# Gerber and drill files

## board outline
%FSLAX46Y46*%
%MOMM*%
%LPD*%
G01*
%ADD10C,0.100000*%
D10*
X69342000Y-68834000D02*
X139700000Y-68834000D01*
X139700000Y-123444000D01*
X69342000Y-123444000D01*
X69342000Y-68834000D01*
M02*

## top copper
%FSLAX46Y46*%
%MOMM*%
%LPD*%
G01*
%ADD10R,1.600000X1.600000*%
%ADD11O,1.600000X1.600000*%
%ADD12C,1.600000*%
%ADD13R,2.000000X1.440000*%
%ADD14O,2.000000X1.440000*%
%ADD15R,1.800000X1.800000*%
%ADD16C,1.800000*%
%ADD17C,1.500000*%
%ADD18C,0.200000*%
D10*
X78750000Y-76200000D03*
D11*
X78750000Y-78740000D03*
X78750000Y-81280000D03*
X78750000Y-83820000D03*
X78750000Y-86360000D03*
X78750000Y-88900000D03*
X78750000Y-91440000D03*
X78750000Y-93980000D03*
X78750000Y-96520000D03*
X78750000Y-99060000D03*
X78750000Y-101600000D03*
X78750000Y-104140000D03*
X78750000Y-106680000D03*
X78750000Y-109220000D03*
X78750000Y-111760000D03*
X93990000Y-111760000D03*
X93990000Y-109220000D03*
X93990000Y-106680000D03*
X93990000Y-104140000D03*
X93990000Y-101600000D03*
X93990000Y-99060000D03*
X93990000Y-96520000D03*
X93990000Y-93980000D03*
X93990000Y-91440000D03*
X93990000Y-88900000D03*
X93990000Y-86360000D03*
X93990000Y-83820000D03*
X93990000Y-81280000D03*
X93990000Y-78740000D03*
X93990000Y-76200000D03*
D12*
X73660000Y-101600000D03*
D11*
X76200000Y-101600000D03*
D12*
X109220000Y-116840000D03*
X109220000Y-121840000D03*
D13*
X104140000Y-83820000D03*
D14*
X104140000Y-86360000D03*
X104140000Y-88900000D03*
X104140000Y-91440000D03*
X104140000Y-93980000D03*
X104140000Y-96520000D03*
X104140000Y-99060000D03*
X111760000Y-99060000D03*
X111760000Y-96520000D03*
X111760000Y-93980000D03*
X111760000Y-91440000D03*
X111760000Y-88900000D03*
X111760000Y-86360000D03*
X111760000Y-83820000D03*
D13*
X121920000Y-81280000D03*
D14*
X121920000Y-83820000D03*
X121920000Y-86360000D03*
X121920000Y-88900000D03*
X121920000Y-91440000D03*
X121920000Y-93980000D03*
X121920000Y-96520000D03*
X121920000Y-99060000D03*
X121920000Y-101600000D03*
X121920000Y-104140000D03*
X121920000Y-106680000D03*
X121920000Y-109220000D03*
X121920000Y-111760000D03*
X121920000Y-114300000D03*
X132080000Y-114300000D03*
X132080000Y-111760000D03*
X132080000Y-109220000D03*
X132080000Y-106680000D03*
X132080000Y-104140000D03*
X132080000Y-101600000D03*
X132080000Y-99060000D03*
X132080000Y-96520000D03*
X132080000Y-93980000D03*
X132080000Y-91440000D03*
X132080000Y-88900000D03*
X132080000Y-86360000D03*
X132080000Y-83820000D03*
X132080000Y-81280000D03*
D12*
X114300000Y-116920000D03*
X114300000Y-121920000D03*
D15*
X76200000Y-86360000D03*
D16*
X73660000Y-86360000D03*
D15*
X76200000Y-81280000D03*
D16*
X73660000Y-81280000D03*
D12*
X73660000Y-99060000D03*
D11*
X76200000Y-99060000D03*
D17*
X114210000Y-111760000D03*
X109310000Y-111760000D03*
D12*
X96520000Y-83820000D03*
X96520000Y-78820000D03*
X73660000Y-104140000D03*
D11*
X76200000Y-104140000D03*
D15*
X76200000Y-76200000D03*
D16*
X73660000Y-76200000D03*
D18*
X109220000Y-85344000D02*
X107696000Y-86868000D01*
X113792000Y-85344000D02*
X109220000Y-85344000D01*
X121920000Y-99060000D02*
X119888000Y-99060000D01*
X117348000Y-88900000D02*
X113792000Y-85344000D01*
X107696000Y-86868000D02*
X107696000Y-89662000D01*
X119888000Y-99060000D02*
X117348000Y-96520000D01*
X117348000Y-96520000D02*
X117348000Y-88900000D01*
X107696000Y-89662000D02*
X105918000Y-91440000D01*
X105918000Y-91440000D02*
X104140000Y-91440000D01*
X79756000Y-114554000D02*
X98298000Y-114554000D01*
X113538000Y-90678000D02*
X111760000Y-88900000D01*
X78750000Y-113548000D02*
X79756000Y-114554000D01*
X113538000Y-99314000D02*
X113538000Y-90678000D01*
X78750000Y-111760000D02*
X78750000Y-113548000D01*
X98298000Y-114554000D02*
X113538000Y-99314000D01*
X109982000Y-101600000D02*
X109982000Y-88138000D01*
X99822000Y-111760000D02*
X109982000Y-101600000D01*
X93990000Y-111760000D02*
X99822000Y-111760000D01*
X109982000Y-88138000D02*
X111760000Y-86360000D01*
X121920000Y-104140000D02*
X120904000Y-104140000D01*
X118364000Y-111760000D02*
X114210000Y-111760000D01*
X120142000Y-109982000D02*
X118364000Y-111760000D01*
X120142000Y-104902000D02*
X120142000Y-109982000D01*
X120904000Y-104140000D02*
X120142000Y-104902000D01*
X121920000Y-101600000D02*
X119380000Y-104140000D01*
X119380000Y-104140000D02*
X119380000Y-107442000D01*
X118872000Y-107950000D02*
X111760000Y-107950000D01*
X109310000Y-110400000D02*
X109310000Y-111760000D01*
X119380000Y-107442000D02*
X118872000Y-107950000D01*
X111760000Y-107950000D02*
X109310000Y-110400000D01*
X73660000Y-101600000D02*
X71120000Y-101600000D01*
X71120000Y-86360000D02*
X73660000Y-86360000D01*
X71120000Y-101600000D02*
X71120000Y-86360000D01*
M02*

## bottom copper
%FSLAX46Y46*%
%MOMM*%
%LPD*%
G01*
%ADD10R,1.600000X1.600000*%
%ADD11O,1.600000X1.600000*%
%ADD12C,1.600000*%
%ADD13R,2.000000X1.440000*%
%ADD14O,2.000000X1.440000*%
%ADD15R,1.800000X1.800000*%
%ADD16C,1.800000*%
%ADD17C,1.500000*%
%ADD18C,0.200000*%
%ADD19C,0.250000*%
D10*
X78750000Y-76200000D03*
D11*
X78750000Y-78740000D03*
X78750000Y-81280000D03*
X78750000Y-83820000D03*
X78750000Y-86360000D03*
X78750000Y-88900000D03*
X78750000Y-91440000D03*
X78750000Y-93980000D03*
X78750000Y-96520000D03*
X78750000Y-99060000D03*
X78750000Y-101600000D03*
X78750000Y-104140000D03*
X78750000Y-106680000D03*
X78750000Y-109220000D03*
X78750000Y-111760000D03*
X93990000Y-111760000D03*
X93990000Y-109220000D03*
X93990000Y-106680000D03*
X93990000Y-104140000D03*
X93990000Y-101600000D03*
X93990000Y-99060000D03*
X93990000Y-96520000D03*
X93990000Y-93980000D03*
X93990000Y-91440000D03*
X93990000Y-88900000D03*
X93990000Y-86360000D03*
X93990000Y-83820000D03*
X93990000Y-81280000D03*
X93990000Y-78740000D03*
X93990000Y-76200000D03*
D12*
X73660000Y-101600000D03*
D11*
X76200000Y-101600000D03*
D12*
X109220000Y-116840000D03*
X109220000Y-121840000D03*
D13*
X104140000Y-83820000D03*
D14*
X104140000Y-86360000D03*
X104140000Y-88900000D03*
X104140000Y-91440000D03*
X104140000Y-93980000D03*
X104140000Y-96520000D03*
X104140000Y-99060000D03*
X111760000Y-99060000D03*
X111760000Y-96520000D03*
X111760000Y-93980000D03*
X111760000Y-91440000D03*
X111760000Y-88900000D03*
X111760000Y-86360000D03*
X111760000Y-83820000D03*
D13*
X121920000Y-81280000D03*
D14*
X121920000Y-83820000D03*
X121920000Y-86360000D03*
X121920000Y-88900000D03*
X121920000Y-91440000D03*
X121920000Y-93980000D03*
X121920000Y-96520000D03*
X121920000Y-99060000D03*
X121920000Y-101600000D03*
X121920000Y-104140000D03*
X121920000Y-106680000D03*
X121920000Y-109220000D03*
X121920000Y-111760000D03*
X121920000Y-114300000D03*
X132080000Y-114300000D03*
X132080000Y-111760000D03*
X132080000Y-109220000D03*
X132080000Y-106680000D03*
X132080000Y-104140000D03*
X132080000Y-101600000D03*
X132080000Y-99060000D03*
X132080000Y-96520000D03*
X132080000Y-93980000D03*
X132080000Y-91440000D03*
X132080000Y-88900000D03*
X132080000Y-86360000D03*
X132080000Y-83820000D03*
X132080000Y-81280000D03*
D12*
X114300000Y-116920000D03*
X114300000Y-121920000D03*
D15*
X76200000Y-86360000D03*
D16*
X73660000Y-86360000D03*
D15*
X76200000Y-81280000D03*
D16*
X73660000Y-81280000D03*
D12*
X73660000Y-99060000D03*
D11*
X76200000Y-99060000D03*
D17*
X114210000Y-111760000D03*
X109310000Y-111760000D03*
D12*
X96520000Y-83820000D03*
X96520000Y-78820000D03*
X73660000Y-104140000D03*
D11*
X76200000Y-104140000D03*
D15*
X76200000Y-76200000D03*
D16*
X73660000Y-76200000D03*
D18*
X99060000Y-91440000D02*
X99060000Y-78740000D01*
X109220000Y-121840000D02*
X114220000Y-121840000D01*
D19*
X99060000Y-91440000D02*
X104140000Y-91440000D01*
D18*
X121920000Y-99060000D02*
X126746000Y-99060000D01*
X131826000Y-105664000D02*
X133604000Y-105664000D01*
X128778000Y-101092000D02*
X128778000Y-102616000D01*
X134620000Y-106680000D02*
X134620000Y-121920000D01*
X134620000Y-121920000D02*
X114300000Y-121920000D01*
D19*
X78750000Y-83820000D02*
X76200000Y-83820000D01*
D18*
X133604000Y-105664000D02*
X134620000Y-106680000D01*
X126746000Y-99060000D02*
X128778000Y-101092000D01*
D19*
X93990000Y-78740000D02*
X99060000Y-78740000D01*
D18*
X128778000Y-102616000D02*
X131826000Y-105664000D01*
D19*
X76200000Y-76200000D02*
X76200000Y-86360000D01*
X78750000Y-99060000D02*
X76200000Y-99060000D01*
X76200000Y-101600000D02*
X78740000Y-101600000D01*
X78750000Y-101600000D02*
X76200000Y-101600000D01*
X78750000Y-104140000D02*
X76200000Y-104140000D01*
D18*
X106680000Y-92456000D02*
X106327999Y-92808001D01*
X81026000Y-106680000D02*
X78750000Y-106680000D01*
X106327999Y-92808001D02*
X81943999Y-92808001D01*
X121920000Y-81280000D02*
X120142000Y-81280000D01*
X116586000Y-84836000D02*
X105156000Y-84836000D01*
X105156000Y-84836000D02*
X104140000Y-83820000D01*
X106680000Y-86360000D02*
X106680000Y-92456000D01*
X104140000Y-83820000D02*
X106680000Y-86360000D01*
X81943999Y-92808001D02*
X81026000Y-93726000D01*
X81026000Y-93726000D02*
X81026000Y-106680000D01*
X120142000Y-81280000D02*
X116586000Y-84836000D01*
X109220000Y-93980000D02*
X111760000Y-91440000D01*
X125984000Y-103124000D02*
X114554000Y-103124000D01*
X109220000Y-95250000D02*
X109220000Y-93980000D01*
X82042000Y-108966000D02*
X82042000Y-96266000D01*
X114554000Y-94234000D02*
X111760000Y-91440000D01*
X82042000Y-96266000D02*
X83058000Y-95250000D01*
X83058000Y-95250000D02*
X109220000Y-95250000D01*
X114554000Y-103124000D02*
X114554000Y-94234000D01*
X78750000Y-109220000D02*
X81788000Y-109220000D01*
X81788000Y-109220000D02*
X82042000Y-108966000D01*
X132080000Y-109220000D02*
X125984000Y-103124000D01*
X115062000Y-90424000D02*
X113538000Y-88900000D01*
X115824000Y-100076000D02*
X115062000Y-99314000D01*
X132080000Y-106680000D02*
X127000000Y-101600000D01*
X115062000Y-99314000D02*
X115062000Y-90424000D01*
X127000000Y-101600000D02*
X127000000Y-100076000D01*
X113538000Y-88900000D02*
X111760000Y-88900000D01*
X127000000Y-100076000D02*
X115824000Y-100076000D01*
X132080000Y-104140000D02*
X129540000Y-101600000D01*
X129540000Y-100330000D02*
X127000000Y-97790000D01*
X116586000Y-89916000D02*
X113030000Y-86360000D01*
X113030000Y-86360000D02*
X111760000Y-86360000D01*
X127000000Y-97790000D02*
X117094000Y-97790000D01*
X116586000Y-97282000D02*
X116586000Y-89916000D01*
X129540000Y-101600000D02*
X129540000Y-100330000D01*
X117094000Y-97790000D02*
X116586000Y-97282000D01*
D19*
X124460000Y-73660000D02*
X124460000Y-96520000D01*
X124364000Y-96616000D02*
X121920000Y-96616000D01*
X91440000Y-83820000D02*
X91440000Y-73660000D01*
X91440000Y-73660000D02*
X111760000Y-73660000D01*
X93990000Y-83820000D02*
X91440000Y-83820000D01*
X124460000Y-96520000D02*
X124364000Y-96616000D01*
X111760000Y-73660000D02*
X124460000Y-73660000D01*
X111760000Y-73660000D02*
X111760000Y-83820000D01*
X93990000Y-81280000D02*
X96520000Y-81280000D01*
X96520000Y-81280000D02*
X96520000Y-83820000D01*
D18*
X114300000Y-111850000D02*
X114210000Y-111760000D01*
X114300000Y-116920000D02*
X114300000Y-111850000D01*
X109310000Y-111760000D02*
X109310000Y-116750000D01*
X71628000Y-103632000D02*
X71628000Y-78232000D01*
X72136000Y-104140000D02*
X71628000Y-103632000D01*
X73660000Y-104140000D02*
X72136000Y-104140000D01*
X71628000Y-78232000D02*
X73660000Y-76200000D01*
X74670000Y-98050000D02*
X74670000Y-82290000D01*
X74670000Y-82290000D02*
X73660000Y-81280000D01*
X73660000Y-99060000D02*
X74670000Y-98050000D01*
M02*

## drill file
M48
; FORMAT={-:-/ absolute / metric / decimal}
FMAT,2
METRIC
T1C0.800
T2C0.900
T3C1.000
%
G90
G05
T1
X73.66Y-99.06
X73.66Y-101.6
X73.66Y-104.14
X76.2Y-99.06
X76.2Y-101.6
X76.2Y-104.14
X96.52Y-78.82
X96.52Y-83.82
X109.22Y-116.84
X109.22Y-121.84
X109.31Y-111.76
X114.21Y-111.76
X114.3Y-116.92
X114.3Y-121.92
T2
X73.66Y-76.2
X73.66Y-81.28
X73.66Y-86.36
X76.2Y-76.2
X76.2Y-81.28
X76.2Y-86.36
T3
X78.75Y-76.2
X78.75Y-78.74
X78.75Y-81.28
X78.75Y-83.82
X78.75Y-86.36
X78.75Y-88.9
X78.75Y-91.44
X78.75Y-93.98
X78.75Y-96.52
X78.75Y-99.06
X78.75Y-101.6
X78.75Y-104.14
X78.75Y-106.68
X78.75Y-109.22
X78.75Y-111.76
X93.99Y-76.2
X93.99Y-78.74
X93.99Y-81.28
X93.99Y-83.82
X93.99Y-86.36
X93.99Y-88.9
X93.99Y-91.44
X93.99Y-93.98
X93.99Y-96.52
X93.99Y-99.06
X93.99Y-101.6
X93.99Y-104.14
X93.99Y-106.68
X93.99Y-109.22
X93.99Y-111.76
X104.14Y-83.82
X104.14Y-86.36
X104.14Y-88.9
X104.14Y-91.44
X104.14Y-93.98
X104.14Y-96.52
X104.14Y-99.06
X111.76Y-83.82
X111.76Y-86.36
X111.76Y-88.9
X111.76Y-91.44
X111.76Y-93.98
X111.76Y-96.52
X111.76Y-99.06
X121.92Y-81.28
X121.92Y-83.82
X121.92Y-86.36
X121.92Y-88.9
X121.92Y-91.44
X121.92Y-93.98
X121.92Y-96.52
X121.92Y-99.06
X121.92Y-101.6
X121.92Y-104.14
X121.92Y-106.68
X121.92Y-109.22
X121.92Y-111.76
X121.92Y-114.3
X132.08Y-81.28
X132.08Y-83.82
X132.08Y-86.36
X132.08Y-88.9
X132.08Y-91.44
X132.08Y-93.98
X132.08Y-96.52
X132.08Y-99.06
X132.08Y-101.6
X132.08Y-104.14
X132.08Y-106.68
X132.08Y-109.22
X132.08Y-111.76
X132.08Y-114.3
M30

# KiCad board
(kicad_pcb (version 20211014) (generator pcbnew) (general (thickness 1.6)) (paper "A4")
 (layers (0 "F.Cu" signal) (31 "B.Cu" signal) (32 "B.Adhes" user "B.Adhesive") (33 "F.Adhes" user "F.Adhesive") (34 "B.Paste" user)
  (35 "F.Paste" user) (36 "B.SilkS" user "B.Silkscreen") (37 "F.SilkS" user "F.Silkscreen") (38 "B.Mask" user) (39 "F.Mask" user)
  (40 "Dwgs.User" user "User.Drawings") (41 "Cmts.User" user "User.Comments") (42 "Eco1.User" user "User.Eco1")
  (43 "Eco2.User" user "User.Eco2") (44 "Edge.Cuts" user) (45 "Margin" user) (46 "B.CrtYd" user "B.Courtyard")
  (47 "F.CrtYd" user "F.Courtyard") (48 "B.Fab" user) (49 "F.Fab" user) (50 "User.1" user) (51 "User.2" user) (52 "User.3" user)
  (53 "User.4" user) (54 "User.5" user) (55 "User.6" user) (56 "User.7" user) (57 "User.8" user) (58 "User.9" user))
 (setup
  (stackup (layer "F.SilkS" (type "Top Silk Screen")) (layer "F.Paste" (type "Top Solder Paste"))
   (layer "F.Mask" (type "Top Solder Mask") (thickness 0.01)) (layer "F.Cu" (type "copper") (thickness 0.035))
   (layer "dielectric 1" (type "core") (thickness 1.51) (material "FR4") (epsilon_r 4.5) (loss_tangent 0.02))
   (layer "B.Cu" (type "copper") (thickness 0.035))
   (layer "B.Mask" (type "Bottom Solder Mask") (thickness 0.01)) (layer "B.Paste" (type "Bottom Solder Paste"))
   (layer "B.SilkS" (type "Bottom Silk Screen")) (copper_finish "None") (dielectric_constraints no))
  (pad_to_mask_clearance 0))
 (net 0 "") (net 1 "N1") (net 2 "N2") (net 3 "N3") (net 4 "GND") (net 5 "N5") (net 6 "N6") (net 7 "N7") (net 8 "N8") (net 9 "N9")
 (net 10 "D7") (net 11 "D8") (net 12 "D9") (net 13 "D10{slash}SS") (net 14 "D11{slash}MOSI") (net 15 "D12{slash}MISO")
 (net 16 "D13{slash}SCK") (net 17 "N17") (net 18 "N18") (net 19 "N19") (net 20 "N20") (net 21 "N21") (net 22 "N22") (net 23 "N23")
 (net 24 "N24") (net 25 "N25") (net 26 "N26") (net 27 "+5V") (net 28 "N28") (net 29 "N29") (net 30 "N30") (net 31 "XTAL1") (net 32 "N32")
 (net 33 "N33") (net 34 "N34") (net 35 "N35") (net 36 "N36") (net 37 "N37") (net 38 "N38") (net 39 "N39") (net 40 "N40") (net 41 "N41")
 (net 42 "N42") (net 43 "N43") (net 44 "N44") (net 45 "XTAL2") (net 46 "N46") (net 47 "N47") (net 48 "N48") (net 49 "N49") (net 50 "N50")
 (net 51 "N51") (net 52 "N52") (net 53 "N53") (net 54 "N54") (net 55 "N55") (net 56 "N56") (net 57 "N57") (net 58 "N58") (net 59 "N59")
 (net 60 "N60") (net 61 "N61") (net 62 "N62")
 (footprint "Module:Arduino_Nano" (layer "F.Cu") (at 78.75 76.2)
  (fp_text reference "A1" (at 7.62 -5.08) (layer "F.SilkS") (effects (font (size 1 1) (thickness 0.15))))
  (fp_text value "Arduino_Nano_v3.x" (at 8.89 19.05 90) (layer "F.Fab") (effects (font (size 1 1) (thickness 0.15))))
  (pad "1" thru_hole rect (at 0 0) (size 1.6 1.6) (drill 1) (layers *.Cu *.Mask) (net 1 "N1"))
  (pad "2" thru_hole oval (at 0 2.54) (size 1.6 1.6) (drill 1) (layers *.Cu *.Mask) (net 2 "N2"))
  (pad "3" thru_hole oval (at 0 5.08) (size 1.6 1.6) (drill 1) (layers *.Cu *.Mask) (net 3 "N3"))
  (pad "4" thru_hole oval (at 0 7.62) (size 1.6 1.6) (drill 1) (layers *.Cu *.Mask) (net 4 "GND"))
  (pad "5" thru_hole oval (at 0 10.16) (size 1.6 1.6) (drill 1) (layers *.Cu *.Mask) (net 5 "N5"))
  (pad "6" thru_hole oval (at 0 12.7) (size 1.6 1.6) (drill 1) (layers *.Cu *.Mask) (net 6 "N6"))
  (pad "7" thru_hole oval (at 0 15.24) (size 1.6 1.6) (drill 1) (layers *.Cu *.Mask) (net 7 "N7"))
  (pad "8" thru_hole oval (at 0 17.78) (size 1.6 1.6) (drill 1) (layers *.Cu *.Mask) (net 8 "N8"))
  (pad "9" thru_hole oval (at 0 20.32) (size 1.6 1.6) (drill 1) (layers *.Cu *.Mask) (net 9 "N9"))
  (pad "10" thru_hole oval (at 0 22.86) (size 1.6 1.6) (drill 1) (layers *.Cu *.Mask) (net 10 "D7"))
  (pad "11" thru_hole oval (at 0 25.4) (size 1.6 1.6) (drill 1) (layers *.Cu *.Mask) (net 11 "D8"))
  (pad "12" thru_hole oval (at 0 27.94) (size 1.6 1.6) (drill 1) (layers *.Cu *.Mask) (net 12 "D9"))
  (pad "13" thru_hole oval (at 0 30.48) (size 1.6 1.6) (drill 1) (layers *.Cu *.Mask) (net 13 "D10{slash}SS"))
  (pad "14" thru_hole oval (at 0 33.02) (size 1.6 1.6) (drill 1) (layers *.Cu *.Mask) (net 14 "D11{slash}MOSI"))
  (pad "15" thru_hole oval (at 0 35.56) (size 1.6 1.6) (drill 1) (layers *.Cu *.Mask) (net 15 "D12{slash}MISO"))
  (pad "16" thru_hole oval (at 15.24 35.56) (size 1.6 1.6) (drill 1) (layers *.Cu *.Mask) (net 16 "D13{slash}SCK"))
  (pad "17" thru_hole oval (at 15.24 33.02) (size 1.6 1.6) (drill 1) (layers *.Cu *.Mask) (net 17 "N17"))
  (pad "18" thru_hole oval (at 15.24 30.48) (size 1.6 1.6) (drill 1) (layers *.Cu *.Mask) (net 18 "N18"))
  (pad "19" thru_hole oval (at 15.24 27.94) (size 1.6 1.6) (drill 1) (layers *.Cu *.Mask) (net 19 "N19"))
  (pad "20" thru_hole oval (at 15.24 25.4) (size 1.6 1.6) (drill 1) (layers *.Cu *.Mask) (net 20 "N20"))
  (pad "21" thru_hole oval (at 15.24 22.86) (size 1.6 1.6) (drill 1) (layers *.Cu *.Mask) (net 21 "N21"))
  (pad "22" thru_hole oval (at 15.24 20.32) (size 1.6 1.6) (drill 1) (layers *.Cu *.Mask) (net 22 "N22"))
  (pad "23" thru_hole oval (at 15.24 17.78) (size 1.6 1.6) (drill 1) (layers *.Cu *.Mask) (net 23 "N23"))
  (pad "24" thru_hole oval (at 15.24 15.24) (size 1.6 1.6) (drill 1) (layers *.Cu *.Mask) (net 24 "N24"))
  (pad "25" thru_hole oval (at 15.24 12.7) (size 1.6 1.6) (drill 1) (layers *.Cu *.Mask) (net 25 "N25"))
  (pad "26" thru_hole oval (at 15.24 10.16) (size 1.6 1.6) (drill 1) (layers *.Cu *.Mask) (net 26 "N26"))
  (pad "27" thru_hole oval (at 15.24 7.62) (size 1.6 1.6) (drill 1) (layers *.Cu *.Mask) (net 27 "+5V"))
  (pad "28" thru_hole oval (at 15.24 5.08) (size 1.6 1.6) (drill 1) (layers *.Cu *.Mask) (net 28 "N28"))
  (pad "29" thru_hole oval (at 15.24 2.54) (size 1.6 1.6) (drill 1) (layers *.Cu *.Mask) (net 4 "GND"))
  (pad "30" thru_hole oval (at 15.24 0) (size 1.6 1.6) (drill 1) (layers *.Cu *.Mask) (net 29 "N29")))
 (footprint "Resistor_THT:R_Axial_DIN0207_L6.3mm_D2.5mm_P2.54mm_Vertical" (layer "F.Cu") (at 73.66 101.6)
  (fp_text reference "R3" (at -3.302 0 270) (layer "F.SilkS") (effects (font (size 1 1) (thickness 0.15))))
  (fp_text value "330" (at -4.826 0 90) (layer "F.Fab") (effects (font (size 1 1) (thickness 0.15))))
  (pad "1" thru_hole circle (at 0 0) (size 1.6 1.6) (drill 0.8) (layers *.Cu *.Mask) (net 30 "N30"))
  (pad "2" thru_hole oval (at 2.54 0) (size 1.6 1.6) (drill 0.8) (layers *.Cu *.Mask) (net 11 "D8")))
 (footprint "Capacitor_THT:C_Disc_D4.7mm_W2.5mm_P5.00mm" (layer "F.Cu") (at 109.22 116.84 -90)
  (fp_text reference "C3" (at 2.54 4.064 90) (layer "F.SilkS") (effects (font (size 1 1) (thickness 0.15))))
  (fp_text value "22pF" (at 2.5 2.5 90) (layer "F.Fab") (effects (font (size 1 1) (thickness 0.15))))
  (pad "1" thru_hole circle (at 0 0 270) (size 1.6 1.6) (drill 0.8) (layers *.Cu *.Mask) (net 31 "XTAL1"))
  (pad "2" thru_hole circle (at 5 0 270) (size 1.6 1.6) (drill 0.8) (layers *.Cu *.Mask) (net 4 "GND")))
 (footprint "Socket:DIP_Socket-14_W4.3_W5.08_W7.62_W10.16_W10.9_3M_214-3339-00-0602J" (layer "F.Cu") (at 104.14 83.82)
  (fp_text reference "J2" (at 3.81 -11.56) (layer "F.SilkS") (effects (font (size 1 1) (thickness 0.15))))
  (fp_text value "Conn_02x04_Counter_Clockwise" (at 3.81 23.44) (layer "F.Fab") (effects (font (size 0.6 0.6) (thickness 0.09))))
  (pad "1" thru_hole rect (at 0 0) (size 2 1.44) (drill 1) (layers *.Cu *.Mask) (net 13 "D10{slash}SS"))
  (pad "2" thru_hole oval (at 0 2.54) (size 2 1.44) (drill 1) (layers *.Cu *.Mask) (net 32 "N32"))
  (pad "3" thru_hole oval (at 0 5.08) (size 2 1.44) (drill 1) (layers *.Cu *.Mask) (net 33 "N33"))
  (pad "4" thru_hole oval (at 0 7.62) (size 2 1.44) (drill 1) (layers *.Cu *.Mask) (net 4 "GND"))
  (pad "5" thru_hole oval (at 0 10.16) (size 2 1.44) (drill 1) (layers *.Cu *.Mask) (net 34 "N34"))
  (pad "6" thru_hole oval (at 0 12.7) (size 2 1.44) (drill 1) (layers *.Cu *.Mask) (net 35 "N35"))
  (pad "7" thru_hole oval (at 0 15.24) (size 2 1.44) (drill 1) (layers *.Cu *.Mask) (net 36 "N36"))
  (pad "8" thru_hole oval (at 7.62 15.24) (size 2 1.44) (drill 1) (layers *.Cu *.Mask) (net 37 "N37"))
  (pad "9" thru_hole oval (at 7.62 12.7) (size 2 1.44) (drill 1) (layers *.Cu *.Mask) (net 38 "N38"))
  (pad "10" thru_hole oval (at 7.62 10.16) (size 2 1.44) (drill 1) (layers *.Cu *.Mask) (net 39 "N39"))
  (pad "11" thru_hole oval (at 7.62 7.62) (size 2 1.44) (drill 1) (layers *.Cu *.Mask) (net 14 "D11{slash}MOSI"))
  (pad "12" thru_hole oval (at 7.62 5.08) (size 2 1.44) (drill 1) (layers *.Cu *.Mask) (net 15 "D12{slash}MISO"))
  (pad "13" thru_hole oval (at 7.62 2.54) (size 2 1.44) (drill 1) (layers *.Cu *.Mask) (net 16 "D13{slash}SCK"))
  (pad "14" thru_hole oval (at 7.62 0) (size 2 1.44) (drill 1) (layers *.Cu *.Mask) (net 27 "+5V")))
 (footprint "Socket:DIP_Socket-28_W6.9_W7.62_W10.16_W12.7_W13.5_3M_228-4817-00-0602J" (layer "F.Cu") (at 121.92 81.28)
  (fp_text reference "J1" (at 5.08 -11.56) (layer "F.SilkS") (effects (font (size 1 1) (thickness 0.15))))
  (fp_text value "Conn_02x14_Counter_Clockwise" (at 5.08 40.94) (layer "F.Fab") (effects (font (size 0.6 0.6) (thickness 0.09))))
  (pad "1" thru_hole rect (at 0 0) (size 2 1.44) (drill 1) (layers *.Cu *.Mask) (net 13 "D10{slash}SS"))
  (pad "2" thru_hole oval (at 0 2.54) (size 2 1.44) (drill 1) (layers *.Cu *.Mask) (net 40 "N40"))
  (pad "3" thru_hole oval (at 0 5.08) (size 2 1.44) (drill 1) (layers *.Cu *.Mask) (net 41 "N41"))
  (pad "4" thru_hole oval (at 0 7.62) (size 2 1.44) (drill 1) (layers *.Cu *.Mask) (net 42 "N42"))
  (pad "5" thru_hole oval (at 0 10.16) (size 2 1.44) (drill 1) (layers *.Cu *.Mask) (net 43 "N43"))
  (pad "6" thru_hole oval (at 0 12.7) (size 2 1.44) (drill 1) (layers *.Cu *.Mask) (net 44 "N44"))
  (pad "7" thru_hole oval (at 0 15.24) (size 2 1.44) (drill 1) (layers *.Cu *.Mask) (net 27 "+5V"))
  (pad "8" thru_hole oval (at 0 17.78) (size 2 1.44) (drill 1) (layers *.Cu *.Mask) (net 4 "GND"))
  (pad "9" thru_hole oval (at 0 20.32) (size 2 1.44) (drill 1) (layers *.Cu *.Mask) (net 31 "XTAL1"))
  (pad "10" thru_hole oval (at 0 22.86) (size 2 1.44) (drill 1) (layers *.Cu *.Mask) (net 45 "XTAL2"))
  (pad "11" thru_hole oval (at 0 25.4) (size 2 1.44) (drill 1) (layers *.Cu *.Mask) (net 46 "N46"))
  (pad "12" thru_hole oval (at 0 27.94) (size 2 1.44) (drill 1) (layers *.Cu *.Mask) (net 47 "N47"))
  (pad "13" thru_hole oval (at 0 30.48) (size 2 1.44) (drill 1) (layers *.Cu *.Mask) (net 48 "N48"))
  (pad "14" thru_hole oval (at 0 33.02) (size 2 1.44) (drill 1) (layers *.Cu *.Mask) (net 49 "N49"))
  (pad "15" thru_hole oval (at 10.16 33.02) (size 2 1.44) (drill 1) (layers *.Cu *.Mask) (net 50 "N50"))
  (pad "16" thru_hole oval (at 10.16 30.48) (size 2 1.44) (drill 1) (layers *.Cu *.Mask) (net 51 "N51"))
  (pad "17" thru_hole oval (at 10.16 27.94) (size 2 1.44) (drill 1) (layers *.Cu *.Mask) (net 14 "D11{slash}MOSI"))
  (pad "18" thru_hole oval (at 10.16 25.4) (size 2 1.44) (drill 1) (layers *.Cu *.Mask) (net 15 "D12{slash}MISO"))
  (pad "19" thru_hole oval (at 10.16 22.86) (size 2 1.44) (drill 1) (layers *.Cu *.Mask) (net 16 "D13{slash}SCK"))
  (pad "20" thru_hole oval (at 10.16 20.32) (size 2 1.44) (drill 1) (layers *.Cu *.Mask) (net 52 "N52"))
  (pad "21" thru_hole oval (at 10.16 17.78) (size 2 1.44) (drill 1) (layers *.Cu *.Mask) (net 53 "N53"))
  (pad "22" thru_hole oval (at 10.16 15.24) (size 2 1.44) (drill 1) (layers *.Cu *.Mask) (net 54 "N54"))
  (pad "23" thru_hole oval (at 10.16 12.7) (size 2 1.44) (drill 1) (layers *.Cu *.Mask) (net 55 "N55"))
  (pad "24" thru_hole oval (at 10.16 10.16) (size 2 1.44) (drill 1) (layers *.Cu *.Mask) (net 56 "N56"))
  (pad "25" thru_hole oval (at 10.16 7.62) (size 2 1.44) (drill 1) (layers *.Cu *.Mask) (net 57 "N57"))
  (pad "26" thru_hole oval (at 10.16 5.08) (size 2 1.44) (drill 1) (layers *.Cu *.Mask) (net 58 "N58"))
  (pad "27" thru_hole oval (at 10.16 2.54) (size 2 1.44) (drill 1) (layers *.Cu *.Mask) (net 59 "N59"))
  (pad "28" thru_hole oval (at 10.16 0) (size 2 1.44) (drill 1) (layers *.Cu *.Mask) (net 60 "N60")))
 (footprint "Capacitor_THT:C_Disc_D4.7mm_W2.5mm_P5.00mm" (layer "F.Cu") (at 114.3 116.92 -90)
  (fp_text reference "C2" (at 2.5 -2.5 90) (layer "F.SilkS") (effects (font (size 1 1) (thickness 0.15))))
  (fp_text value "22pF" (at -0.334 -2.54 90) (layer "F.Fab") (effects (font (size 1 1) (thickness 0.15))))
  (pad "1" thru_hole circle (at 0 0 270) (size 1.6 1.6) (drill 0.8) (layers *.Cu *.Mask) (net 45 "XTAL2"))
  (pad "2" thru_hole circle (at 5 0 270) (size 1.6 1.6) (drill 0.8) (layers *.Cu *.Mask) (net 4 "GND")))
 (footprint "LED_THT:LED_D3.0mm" (layer "F.Cu") (at 76.2 86.36 180)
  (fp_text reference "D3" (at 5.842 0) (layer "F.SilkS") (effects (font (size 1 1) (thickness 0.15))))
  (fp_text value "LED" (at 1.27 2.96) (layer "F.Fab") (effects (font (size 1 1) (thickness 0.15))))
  (pad "1" thru_hole rect (at 0 0 180) (size 1.8 1.8) (drill 0.9) (layers *.Cu *.Mask) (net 4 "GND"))
  (pad "2" thru_hole circle (at 2.54 0 180) (size 1.8 1.8) (drill 0.9) (layers *.Cu *.Mask) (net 30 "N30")))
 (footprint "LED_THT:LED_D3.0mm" (layer "F.Cu") (at 76.2 81.28 180)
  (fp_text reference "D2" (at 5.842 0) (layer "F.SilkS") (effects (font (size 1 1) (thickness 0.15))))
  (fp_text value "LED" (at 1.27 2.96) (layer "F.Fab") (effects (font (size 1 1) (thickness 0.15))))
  (pad "1" thru_hole rect (at 0 0 180) (size 1.8 1.8) (drill 0.9) (layers *.Cu *.Mask) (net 4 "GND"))
  (pad "2" thru_hole circle (at 2.54 0 180) (size 1.8 1.8) (drill 0.9) (layers *.Cu *.Mask) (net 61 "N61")))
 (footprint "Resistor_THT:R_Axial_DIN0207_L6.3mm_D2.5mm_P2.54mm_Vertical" (layer "F.Cu") (at 73.66 99.06)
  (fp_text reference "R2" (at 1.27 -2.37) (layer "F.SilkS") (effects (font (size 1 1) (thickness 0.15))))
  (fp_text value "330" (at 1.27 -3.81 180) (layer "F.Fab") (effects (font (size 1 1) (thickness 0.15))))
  (pad "1" thru_hole circle (at 0 0) (size 1.6 1.6) (drill 0.8) (layers *.Cu *.Mask) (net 61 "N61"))
  (pad "2" thru_hole oval (at 2.54 0) (size 1.6 1.6) (drill 0.8) (layers *.Cu *.Mask) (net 10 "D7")))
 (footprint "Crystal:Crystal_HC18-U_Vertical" (layer "F.Cu") (at 114.21 111.76 180)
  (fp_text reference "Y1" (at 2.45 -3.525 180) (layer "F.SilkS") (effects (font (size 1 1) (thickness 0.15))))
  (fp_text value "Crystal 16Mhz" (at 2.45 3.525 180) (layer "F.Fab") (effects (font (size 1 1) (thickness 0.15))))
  (pad "1" thru_hole circle (at 0 0 180) (size 1.5 1.5) (drill 0.8) (layers *.Cu *.Mask) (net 45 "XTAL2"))
  (pad "2" thru_hole circle (at 4.9 0 180) (size 1.5 1.5) (drill 0.8) (layers *.Cu *.Mask) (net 31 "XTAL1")))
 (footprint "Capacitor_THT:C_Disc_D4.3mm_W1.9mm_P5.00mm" (layer "F.Cu") (at 96.52 83.82 90)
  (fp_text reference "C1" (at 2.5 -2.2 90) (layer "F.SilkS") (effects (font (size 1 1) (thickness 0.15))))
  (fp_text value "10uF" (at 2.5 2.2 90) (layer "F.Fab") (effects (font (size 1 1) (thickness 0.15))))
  (pad "1" thru_hole circle (at 0 0 90) (size 1.6 1.6) (drill 0.8) (layers *.Cu *.Mask) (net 28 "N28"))
  (pad "2" thru_hole circle (at 5 0 90) (size 1.6 1.6) (drill 0.8) (layers *.Cu *.Mask) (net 4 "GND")))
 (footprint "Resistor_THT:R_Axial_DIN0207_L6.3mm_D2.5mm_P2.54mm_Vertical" (layer "F.Cu") (at 73.66 104.14)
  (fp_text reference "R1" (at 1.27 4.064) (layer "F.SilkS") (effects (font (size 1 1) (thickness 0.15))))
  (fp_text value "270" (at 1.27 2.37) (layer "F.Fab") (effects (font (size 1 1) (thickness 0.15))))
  (pad "1" thru_hole circle (at 0 0) (size 1.6 1.6) (drill 0.8) (layers *.Cu *.Mask) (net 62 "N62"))
  (pad "2" thru_hole oval (at 2.54 0) (size 1.6 1.6) (drill 0.8) (layers *.Cu *.Mask) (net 12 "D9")))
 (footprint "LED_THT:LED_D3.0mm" (layer "F.Cu") (at 76.2 76.2 180)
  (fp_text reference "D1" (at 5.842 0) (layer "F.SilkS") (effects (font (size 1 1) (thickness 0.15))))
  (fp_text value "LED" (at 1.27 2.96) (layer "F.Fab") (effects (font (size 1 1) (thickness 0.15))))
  (pad "1" thru_hole rect (at 0 0 180) (size 1.8 1.8) (drill 0.9) (layers *.Cu *.Mask) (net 4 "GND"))
  (pad "2" thru_hole circle (at 2.54 0 180) (size 1.8 1.8) (drill 0.9) (layers *.Cu *.Mask) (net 62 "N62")))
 (gr_rect (start 139.7 68.834) (end 69.342 123.444) (layer "Edge.Cuts") (width 0.1) (fill none))
 (segment (start 109.22 85.344) (end 107.696 86.868) (width 0.2) (layer "F.Cu") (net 4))
 (segment (start 113.792 85.344) (end 109.22 85.344) (width 0.2) (layer "F.Cu") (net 4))
 (segment (start 121.92 99.06) (end 119.888 99.06) (width 0.2) (layer "F.Cu") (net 4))
 (segment (start 117.348 88.9) (end 113.792 85.344) (width 0.2) (layer "F.Cu") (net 4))
 (segment (start 107.696 86.868) (end 107.696 89.662) (width 0.2) (layer "F.Cu") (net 4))
 (segment (start 119.888 99.06) (end 117.348 96.52) (width 0.2) (layer "F.Cu") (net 4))
 (segment (start 117.348 96.52) (end 117.348 88.9) (width 0.2) (layer "F.Cu") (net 4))
 (segment (start 107.696 89.662) (end 105.918 91.44) (width 0.2) (layer "F.Cu") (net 4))
 (segment (start 105.918 91.44) (end 104.14 91.44) (width 0.2) (layer "F.Cu") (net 4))
 (segment (start 99.06 91.44) (end 99.06 78.74) (width 0.2) (layer "B.Cu") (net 4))
 (segment (start 109.22 121.84) (end 114.22 121.84) (width 0.2) (layer "B.Cu") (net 4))
 (segment (start 99.06 91.44) (end 104.14 91.44) (width 0.25) (layer "B.Cu") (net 4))
 (segment (start 121.92 99.06) (end 126.746 99.06) (width 0.2) (layer "B.Cu") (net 4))
 (segment (start 131.826 105.664) (end 133.604 105.664) (width 0.2) (layer "B.Cu") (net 4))
 (segment (start 128.778 101.092) (end 128.778 102.616) (width 0.2) (layer "B.Cu") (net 4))
 (segment (start 134.62 106.68) (end 134.62 121.92) (width 0.2) (layer "B.Cu") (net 4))
 (segment (start 134.62 121.92) (end 114.3 121.92) (width 0.2) (layer "B.Cu") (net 4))
 (segment (start 78.75 83.82) (end 76.2 83.82) (width 0.25) (layer "B.Cu") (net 4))
 (segment (start 133.604 105.664) (end 134.62 106.68) (width 0.2) (layer "B.Cu") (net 4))
 (segment (start 126.746 99.06) (end 128.778 101.092) (width 0.2) (layer "B.Cu") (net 4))
 (segment (start 93.99 78.74) (end 99.06 78.74) (width 0.25) (layer "B.Cu") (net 4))
 (segment (start 128.778 102.616) (end 131.826 105.664) (width 0.2) (layer "B.Cu") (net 4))
 (segment (start 76.2 76.2) (end 76.2 86.36) (width 0.25) (layer "B.Cu") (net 4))
 (segment (start 78.75 99.06) (end 76.2 99.06) (width 0.25) (layer "B.Cu") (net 10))
 (segment (start 76.2 101.6) (end 78.74 101.6) (width 0.25) (layer "B.Cu") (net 11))
 (segment (start 78.75 101.6) (end 76.2 101.6) (width 0.25) (layer "B.Cu") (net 11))
 (segment (start 78.75 104.14) (end 76.2 104.14) (width 0.25) (layer "B.Cu") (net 12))
 (segment (start 106.68 92.456) (end 106.327999 92.808001) (width 0.2) (layer "B.Cu") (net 13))
 (segment (start 81.026 106.68) (end 78.75 106.68) (width 0.2) (layer "B.Cu") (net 13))
 (segment (start 106.327999 92.808001) (end 81.943999 92.808001) (width 0.2) (layer "B.Cu") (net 13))
 (segment (start 121.92 81.28) (end 120.142 81.28) (width 0.2) (layer "B.Cu") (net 13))
 (segment (start 116.586 84.836) (end 105.156 84.836) (width 0.2) (layer "B.Cu") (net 13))
 (segment (start 105.156 84.836) (end 104.14 83.82) (width 0.2) (layer "B.Cu") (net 13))
 (segment (start 106.68 86.36) (end 106.68 92.456) (width 0.2) (layer "B.Cu") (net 13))
 (segment (start 104.14 83.82) (end 106.68 86.36) (width 0.2) (layer "B.Cu") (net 13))
 (segment (start 81.943999 92.808001) (end 81.026 93.726) (width 0.2) (layer "B.Cu") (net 13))
 (segment (start 81.026 93.726) (end 81.026 106.68) (width 0.2) (layer "B.Cu") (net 13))
 (segment (start 120.142 81.28) (end 116.586 84.836) (width 0.2) (layer "B.Cu") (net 13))
 (segment (start 109.22 93.98) (end 111.76 91.44) (width 0.2) (layer "B.Cu") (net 14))
 (segment (start 125.984 103.124) (end 114.554 103.124) (width 0.2) (layer "B.Cu") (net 14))
 (segment (start 109.22 95.25) (end 109.22 93.98) (width 0.2) (layer "B.Cu") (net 14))
 (segment (start 82.042 108.966) (end 82.042 96.266) (width 0.2) (layer "B.Cu") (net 14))
 (segment (start 114.554 94.234) (end 111.76 91.44) (width 0.2) (layer "B.Cu") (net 14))
 (segment (start 82.042 96.266) (end 83.058 95.25) (width 0.2) (layer "B.Cu") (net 14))
 (segment (start 83.058 95.25) (end 109.22 95.25) (width 0.2) (layer "B.Cu") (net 14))
 (segment (start 114.554 103.124) (end 114.554 94.234) (width 0.2) (layer "B.Cu") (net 14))
 (segment (start 78.75 109.22) (end 81.788 109.22) (width 0.2) (layer "B.Cu") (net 14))
 (segment (start 81.788 109.22) (end 82.042 108.966) (width 0.2) (layer "B.Cu") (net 14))
 (segment (start 132.08 109.22) (end 125.984 103.124) (width 0.2) (layer "B.Cu") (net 14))
 (segment (start 79.756 114.554) (end 98.298 114.554) (width 0.2) (layer "F.Cu") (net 15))
 (segment (start 113.538 90.678) (end 111.76 88.9) (width 0.2) (layer "F.Cu") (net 15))
 (segment (start 78.75 113.548) (end 79.756 114.554) (width 0.2) (layer "F.Cu") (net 15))
 (segment (start 113.538 99.314) (end 113.538 90.678) (width 0.2) (layer "F.Cu") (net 15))
 (segment (start 78.75 111.76) (end 78.75 113.548) (width 0.2) (layer "F.Cu") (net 15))
 (segment (start 98.298 114.554) (end 113.538 99.314) (width 0.2) (layer "F.Cu") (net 15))
 (segment (start 115.062 90.424) (end 113.538 88.9) (width 0.2) (layer "B.Cu") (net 15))
 (segment (start 115.824 100.076) (end 115.062 99.314) (width 0.2) (layer "B.Cu") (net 15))
 (segment (start 132.08 106.68) (end 127 101.6) (width 0.2) (layer "B.Cu") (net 15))
 (segment (start 115.062 99.314) (end 115.062 90.424) (width 0.2) (layer "B.Cu") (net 15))
 (segment (start 127 101.6) (end 127 100.076) (width 0.2) (layer "B.Cu") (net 15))
 (segment (start 113.538 88.9) (end 111.76 88.9) (width 0.2) (layer "B.Cu") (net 15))
 (segment (start 127 100.076) (end 115.824 100.076) (width 0.2) (layer "B.Cu") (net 15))
 (segment (start 109.982 101.6) (end 109.982 88.138) (width 0.2) (layer "F.Cu") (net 16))
 (segment (start 99.822 111.76) (end 109.982 101.6) (width 0.2) (layer "F.Cu") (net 16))
 (segment (start 93.99 111.76) (end 99.822 111.76) (width 0.2) (layer "F.Cu") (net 16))
 (segment (start 109.982 88.138) (end 111.76 86.36) (width 0.2) (layer "F.Cu") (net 16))
 (segment (start 132.08 104.14) (end 129.54 101.6) (width 0.2) (layer "B.Cu") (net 16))
 (segment (start 129.54 100.33) (end 127 97.79) (width 0.2) (layer "B.Cu") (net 16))
 (segment (start 116.586 89.916) (end 113.03 86.36) (width 0.2) (layer "B.Cu") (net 16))
 (segment (start 113.03 86.36) (end 111.76 86.36) (width 0.2) (layer "B.Cu") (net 16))
 (segment (start 127 97.79) (end 117.094 97.79) (width 0.2) (layer "B.Cu") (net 16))
 (segment (start 116.586 97.282) (end 116.586 89.916) (width 0.2) (layer "B.Cu") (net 16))
 (segment (start 129.54 101.6) (end 129.54 100.33) (width 0.2) (layer "B.Cu") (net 16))
 (segment (start 117.094 97.79) (end 116.586 97.282) (width 0.2) (layer "B.Cu") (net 16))
 (segment (start 124.46 73.66) (end 124.46 96.52) (width 0.25) (layer "B.Cu") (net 27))
 (segment (start 124.364 96.616) (end 121.92 96.616) (width 0.25) (layer "B.Cu") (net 27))
 (segment (start 91.44 83.82) (end 91.44 73.66) (width 0.25) (layer "B.Cu") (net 27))
 (segment (start 91.44 73.66) (end 111.76 73.66) (width 0.25) (layer "B.Cu") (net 27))
 (segment (start 93.99 83.82) (end 91.44 83.82) (width 0.25) (layer "B.Cu") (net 27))
 (segment (start 124.46 96.52) (end 124.364 96.616) (width 0.25) (layer "B.Cu") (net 27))
 (segment (start 111.76 73.66) (end 124.46 73.66) (width 0.25) (layer "B.Cu") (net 27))
 (segment (start 111.76 73.66) (end 111.76 83.82) (width 0.25) (layer "B.Cu") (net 27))
 (segment (start 93.99 81.28) (end 96.52 81.28) (width 0.25) (layer "B.Cu") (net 28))
 (segment (start 96.52 81.28) (end 96.52 83.82) (width 0.25) (layer "B.Cu") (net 28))
 (segment (start 121.92 104.14) (end 120.904 104.14) (width 0.2) (layer "F.Cu") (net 45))
 (segment (start 118.364 111.76) (end 114.21 111.76) (width 0.2) (layer "F.Cu") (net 45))
 (segment (start 120.142 109.982) (end 118.364 111.76) (width 0.2) (layer "F.Cu") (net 45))
 (segment (start 120.142 104.902) (end 120.142 109.982) (width 0.2) (layer "F.Cu") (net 45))
 (segment (start 120.904 104.14) (end 120.142 104.902) (width 0.2) (layer "F.Cu") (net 45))
 (segment (start 114.3 111.85) (end 114.21 111.76) (width 0.2) (layer "B.Cu") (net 45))
 (segment (start 114.3 116.92) (end 114.3 111.85) (width 0.2) (layer "B.Cu") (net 45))
 (segment (start 121.92 101.6) (end 119.38 104.14) (width 0.2) (layer "F.Cu") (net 31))
 (segment (start 119.38 104.14) (end 119.38 107.442) (width 0.2) (layer "F.Cu") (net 31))
 (segment (start 118.872 107.95) (end 111.76 107.95) (width 0.2) (layer "F.Cu") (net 31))
 (segment (start 109.31 110.4) (end 109.31 111.76) (width 0.2) (layer "F.Cu") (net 31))
 (segment (start 119.38 107.442) (end 118.872 107.95) (width 0.2) (layer "F.Cu") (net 31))
 (segment (start 111.76 107.95) (end 109.31 110.4) (width 0.2) (layer "F.Cu") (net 31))
 (segment (start 109.31 111.76) (end 109.31 116.75) (width 0.2) (layer "B.Cu") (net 31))
 (segment (start 71.628 103.632) (end 71.628 78.232) (width 0.2) (layer "B.Cu") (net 62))
 (segment (start 72.136 104.14) (end 71.628 103.632) (width 0.2) (layer "B.Cu") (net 62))
 (segment (start 73.66 104.14) (end 72.136 104.14) (width 0.2) (layer "B.Cu") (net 62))
 (segment (start 71.628 78.232) (end 73.66 76.2) (width 0.2) (layer "B.Cu") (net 62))
 (segment (start 74.67 98.05) (end 74.67 82.29) (width 0.2) (layer "B.Cu") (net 61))
 (segment (start 74.67 82.29) (end 73.66 81.28) (width 0.2) (layer "B.Cu") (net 61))
 (segment (start 73.66 99.06) (end 74.67 98.05) (width 0.2) (layer "B.Cu") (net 61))
 (segment (start 73.66 101.6) (end 71.12 101.6) (width 0.2) (layer "F.Cu") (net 30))
 (segment (start 71.12 86.36) (end 73.66 86.36) (width 0.2) (layer "F.Cu") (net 30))
 (segment (start 71.12 101.6) (end 71.12 86.36) (width 0.2) (layer "F.Cu") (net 30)))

